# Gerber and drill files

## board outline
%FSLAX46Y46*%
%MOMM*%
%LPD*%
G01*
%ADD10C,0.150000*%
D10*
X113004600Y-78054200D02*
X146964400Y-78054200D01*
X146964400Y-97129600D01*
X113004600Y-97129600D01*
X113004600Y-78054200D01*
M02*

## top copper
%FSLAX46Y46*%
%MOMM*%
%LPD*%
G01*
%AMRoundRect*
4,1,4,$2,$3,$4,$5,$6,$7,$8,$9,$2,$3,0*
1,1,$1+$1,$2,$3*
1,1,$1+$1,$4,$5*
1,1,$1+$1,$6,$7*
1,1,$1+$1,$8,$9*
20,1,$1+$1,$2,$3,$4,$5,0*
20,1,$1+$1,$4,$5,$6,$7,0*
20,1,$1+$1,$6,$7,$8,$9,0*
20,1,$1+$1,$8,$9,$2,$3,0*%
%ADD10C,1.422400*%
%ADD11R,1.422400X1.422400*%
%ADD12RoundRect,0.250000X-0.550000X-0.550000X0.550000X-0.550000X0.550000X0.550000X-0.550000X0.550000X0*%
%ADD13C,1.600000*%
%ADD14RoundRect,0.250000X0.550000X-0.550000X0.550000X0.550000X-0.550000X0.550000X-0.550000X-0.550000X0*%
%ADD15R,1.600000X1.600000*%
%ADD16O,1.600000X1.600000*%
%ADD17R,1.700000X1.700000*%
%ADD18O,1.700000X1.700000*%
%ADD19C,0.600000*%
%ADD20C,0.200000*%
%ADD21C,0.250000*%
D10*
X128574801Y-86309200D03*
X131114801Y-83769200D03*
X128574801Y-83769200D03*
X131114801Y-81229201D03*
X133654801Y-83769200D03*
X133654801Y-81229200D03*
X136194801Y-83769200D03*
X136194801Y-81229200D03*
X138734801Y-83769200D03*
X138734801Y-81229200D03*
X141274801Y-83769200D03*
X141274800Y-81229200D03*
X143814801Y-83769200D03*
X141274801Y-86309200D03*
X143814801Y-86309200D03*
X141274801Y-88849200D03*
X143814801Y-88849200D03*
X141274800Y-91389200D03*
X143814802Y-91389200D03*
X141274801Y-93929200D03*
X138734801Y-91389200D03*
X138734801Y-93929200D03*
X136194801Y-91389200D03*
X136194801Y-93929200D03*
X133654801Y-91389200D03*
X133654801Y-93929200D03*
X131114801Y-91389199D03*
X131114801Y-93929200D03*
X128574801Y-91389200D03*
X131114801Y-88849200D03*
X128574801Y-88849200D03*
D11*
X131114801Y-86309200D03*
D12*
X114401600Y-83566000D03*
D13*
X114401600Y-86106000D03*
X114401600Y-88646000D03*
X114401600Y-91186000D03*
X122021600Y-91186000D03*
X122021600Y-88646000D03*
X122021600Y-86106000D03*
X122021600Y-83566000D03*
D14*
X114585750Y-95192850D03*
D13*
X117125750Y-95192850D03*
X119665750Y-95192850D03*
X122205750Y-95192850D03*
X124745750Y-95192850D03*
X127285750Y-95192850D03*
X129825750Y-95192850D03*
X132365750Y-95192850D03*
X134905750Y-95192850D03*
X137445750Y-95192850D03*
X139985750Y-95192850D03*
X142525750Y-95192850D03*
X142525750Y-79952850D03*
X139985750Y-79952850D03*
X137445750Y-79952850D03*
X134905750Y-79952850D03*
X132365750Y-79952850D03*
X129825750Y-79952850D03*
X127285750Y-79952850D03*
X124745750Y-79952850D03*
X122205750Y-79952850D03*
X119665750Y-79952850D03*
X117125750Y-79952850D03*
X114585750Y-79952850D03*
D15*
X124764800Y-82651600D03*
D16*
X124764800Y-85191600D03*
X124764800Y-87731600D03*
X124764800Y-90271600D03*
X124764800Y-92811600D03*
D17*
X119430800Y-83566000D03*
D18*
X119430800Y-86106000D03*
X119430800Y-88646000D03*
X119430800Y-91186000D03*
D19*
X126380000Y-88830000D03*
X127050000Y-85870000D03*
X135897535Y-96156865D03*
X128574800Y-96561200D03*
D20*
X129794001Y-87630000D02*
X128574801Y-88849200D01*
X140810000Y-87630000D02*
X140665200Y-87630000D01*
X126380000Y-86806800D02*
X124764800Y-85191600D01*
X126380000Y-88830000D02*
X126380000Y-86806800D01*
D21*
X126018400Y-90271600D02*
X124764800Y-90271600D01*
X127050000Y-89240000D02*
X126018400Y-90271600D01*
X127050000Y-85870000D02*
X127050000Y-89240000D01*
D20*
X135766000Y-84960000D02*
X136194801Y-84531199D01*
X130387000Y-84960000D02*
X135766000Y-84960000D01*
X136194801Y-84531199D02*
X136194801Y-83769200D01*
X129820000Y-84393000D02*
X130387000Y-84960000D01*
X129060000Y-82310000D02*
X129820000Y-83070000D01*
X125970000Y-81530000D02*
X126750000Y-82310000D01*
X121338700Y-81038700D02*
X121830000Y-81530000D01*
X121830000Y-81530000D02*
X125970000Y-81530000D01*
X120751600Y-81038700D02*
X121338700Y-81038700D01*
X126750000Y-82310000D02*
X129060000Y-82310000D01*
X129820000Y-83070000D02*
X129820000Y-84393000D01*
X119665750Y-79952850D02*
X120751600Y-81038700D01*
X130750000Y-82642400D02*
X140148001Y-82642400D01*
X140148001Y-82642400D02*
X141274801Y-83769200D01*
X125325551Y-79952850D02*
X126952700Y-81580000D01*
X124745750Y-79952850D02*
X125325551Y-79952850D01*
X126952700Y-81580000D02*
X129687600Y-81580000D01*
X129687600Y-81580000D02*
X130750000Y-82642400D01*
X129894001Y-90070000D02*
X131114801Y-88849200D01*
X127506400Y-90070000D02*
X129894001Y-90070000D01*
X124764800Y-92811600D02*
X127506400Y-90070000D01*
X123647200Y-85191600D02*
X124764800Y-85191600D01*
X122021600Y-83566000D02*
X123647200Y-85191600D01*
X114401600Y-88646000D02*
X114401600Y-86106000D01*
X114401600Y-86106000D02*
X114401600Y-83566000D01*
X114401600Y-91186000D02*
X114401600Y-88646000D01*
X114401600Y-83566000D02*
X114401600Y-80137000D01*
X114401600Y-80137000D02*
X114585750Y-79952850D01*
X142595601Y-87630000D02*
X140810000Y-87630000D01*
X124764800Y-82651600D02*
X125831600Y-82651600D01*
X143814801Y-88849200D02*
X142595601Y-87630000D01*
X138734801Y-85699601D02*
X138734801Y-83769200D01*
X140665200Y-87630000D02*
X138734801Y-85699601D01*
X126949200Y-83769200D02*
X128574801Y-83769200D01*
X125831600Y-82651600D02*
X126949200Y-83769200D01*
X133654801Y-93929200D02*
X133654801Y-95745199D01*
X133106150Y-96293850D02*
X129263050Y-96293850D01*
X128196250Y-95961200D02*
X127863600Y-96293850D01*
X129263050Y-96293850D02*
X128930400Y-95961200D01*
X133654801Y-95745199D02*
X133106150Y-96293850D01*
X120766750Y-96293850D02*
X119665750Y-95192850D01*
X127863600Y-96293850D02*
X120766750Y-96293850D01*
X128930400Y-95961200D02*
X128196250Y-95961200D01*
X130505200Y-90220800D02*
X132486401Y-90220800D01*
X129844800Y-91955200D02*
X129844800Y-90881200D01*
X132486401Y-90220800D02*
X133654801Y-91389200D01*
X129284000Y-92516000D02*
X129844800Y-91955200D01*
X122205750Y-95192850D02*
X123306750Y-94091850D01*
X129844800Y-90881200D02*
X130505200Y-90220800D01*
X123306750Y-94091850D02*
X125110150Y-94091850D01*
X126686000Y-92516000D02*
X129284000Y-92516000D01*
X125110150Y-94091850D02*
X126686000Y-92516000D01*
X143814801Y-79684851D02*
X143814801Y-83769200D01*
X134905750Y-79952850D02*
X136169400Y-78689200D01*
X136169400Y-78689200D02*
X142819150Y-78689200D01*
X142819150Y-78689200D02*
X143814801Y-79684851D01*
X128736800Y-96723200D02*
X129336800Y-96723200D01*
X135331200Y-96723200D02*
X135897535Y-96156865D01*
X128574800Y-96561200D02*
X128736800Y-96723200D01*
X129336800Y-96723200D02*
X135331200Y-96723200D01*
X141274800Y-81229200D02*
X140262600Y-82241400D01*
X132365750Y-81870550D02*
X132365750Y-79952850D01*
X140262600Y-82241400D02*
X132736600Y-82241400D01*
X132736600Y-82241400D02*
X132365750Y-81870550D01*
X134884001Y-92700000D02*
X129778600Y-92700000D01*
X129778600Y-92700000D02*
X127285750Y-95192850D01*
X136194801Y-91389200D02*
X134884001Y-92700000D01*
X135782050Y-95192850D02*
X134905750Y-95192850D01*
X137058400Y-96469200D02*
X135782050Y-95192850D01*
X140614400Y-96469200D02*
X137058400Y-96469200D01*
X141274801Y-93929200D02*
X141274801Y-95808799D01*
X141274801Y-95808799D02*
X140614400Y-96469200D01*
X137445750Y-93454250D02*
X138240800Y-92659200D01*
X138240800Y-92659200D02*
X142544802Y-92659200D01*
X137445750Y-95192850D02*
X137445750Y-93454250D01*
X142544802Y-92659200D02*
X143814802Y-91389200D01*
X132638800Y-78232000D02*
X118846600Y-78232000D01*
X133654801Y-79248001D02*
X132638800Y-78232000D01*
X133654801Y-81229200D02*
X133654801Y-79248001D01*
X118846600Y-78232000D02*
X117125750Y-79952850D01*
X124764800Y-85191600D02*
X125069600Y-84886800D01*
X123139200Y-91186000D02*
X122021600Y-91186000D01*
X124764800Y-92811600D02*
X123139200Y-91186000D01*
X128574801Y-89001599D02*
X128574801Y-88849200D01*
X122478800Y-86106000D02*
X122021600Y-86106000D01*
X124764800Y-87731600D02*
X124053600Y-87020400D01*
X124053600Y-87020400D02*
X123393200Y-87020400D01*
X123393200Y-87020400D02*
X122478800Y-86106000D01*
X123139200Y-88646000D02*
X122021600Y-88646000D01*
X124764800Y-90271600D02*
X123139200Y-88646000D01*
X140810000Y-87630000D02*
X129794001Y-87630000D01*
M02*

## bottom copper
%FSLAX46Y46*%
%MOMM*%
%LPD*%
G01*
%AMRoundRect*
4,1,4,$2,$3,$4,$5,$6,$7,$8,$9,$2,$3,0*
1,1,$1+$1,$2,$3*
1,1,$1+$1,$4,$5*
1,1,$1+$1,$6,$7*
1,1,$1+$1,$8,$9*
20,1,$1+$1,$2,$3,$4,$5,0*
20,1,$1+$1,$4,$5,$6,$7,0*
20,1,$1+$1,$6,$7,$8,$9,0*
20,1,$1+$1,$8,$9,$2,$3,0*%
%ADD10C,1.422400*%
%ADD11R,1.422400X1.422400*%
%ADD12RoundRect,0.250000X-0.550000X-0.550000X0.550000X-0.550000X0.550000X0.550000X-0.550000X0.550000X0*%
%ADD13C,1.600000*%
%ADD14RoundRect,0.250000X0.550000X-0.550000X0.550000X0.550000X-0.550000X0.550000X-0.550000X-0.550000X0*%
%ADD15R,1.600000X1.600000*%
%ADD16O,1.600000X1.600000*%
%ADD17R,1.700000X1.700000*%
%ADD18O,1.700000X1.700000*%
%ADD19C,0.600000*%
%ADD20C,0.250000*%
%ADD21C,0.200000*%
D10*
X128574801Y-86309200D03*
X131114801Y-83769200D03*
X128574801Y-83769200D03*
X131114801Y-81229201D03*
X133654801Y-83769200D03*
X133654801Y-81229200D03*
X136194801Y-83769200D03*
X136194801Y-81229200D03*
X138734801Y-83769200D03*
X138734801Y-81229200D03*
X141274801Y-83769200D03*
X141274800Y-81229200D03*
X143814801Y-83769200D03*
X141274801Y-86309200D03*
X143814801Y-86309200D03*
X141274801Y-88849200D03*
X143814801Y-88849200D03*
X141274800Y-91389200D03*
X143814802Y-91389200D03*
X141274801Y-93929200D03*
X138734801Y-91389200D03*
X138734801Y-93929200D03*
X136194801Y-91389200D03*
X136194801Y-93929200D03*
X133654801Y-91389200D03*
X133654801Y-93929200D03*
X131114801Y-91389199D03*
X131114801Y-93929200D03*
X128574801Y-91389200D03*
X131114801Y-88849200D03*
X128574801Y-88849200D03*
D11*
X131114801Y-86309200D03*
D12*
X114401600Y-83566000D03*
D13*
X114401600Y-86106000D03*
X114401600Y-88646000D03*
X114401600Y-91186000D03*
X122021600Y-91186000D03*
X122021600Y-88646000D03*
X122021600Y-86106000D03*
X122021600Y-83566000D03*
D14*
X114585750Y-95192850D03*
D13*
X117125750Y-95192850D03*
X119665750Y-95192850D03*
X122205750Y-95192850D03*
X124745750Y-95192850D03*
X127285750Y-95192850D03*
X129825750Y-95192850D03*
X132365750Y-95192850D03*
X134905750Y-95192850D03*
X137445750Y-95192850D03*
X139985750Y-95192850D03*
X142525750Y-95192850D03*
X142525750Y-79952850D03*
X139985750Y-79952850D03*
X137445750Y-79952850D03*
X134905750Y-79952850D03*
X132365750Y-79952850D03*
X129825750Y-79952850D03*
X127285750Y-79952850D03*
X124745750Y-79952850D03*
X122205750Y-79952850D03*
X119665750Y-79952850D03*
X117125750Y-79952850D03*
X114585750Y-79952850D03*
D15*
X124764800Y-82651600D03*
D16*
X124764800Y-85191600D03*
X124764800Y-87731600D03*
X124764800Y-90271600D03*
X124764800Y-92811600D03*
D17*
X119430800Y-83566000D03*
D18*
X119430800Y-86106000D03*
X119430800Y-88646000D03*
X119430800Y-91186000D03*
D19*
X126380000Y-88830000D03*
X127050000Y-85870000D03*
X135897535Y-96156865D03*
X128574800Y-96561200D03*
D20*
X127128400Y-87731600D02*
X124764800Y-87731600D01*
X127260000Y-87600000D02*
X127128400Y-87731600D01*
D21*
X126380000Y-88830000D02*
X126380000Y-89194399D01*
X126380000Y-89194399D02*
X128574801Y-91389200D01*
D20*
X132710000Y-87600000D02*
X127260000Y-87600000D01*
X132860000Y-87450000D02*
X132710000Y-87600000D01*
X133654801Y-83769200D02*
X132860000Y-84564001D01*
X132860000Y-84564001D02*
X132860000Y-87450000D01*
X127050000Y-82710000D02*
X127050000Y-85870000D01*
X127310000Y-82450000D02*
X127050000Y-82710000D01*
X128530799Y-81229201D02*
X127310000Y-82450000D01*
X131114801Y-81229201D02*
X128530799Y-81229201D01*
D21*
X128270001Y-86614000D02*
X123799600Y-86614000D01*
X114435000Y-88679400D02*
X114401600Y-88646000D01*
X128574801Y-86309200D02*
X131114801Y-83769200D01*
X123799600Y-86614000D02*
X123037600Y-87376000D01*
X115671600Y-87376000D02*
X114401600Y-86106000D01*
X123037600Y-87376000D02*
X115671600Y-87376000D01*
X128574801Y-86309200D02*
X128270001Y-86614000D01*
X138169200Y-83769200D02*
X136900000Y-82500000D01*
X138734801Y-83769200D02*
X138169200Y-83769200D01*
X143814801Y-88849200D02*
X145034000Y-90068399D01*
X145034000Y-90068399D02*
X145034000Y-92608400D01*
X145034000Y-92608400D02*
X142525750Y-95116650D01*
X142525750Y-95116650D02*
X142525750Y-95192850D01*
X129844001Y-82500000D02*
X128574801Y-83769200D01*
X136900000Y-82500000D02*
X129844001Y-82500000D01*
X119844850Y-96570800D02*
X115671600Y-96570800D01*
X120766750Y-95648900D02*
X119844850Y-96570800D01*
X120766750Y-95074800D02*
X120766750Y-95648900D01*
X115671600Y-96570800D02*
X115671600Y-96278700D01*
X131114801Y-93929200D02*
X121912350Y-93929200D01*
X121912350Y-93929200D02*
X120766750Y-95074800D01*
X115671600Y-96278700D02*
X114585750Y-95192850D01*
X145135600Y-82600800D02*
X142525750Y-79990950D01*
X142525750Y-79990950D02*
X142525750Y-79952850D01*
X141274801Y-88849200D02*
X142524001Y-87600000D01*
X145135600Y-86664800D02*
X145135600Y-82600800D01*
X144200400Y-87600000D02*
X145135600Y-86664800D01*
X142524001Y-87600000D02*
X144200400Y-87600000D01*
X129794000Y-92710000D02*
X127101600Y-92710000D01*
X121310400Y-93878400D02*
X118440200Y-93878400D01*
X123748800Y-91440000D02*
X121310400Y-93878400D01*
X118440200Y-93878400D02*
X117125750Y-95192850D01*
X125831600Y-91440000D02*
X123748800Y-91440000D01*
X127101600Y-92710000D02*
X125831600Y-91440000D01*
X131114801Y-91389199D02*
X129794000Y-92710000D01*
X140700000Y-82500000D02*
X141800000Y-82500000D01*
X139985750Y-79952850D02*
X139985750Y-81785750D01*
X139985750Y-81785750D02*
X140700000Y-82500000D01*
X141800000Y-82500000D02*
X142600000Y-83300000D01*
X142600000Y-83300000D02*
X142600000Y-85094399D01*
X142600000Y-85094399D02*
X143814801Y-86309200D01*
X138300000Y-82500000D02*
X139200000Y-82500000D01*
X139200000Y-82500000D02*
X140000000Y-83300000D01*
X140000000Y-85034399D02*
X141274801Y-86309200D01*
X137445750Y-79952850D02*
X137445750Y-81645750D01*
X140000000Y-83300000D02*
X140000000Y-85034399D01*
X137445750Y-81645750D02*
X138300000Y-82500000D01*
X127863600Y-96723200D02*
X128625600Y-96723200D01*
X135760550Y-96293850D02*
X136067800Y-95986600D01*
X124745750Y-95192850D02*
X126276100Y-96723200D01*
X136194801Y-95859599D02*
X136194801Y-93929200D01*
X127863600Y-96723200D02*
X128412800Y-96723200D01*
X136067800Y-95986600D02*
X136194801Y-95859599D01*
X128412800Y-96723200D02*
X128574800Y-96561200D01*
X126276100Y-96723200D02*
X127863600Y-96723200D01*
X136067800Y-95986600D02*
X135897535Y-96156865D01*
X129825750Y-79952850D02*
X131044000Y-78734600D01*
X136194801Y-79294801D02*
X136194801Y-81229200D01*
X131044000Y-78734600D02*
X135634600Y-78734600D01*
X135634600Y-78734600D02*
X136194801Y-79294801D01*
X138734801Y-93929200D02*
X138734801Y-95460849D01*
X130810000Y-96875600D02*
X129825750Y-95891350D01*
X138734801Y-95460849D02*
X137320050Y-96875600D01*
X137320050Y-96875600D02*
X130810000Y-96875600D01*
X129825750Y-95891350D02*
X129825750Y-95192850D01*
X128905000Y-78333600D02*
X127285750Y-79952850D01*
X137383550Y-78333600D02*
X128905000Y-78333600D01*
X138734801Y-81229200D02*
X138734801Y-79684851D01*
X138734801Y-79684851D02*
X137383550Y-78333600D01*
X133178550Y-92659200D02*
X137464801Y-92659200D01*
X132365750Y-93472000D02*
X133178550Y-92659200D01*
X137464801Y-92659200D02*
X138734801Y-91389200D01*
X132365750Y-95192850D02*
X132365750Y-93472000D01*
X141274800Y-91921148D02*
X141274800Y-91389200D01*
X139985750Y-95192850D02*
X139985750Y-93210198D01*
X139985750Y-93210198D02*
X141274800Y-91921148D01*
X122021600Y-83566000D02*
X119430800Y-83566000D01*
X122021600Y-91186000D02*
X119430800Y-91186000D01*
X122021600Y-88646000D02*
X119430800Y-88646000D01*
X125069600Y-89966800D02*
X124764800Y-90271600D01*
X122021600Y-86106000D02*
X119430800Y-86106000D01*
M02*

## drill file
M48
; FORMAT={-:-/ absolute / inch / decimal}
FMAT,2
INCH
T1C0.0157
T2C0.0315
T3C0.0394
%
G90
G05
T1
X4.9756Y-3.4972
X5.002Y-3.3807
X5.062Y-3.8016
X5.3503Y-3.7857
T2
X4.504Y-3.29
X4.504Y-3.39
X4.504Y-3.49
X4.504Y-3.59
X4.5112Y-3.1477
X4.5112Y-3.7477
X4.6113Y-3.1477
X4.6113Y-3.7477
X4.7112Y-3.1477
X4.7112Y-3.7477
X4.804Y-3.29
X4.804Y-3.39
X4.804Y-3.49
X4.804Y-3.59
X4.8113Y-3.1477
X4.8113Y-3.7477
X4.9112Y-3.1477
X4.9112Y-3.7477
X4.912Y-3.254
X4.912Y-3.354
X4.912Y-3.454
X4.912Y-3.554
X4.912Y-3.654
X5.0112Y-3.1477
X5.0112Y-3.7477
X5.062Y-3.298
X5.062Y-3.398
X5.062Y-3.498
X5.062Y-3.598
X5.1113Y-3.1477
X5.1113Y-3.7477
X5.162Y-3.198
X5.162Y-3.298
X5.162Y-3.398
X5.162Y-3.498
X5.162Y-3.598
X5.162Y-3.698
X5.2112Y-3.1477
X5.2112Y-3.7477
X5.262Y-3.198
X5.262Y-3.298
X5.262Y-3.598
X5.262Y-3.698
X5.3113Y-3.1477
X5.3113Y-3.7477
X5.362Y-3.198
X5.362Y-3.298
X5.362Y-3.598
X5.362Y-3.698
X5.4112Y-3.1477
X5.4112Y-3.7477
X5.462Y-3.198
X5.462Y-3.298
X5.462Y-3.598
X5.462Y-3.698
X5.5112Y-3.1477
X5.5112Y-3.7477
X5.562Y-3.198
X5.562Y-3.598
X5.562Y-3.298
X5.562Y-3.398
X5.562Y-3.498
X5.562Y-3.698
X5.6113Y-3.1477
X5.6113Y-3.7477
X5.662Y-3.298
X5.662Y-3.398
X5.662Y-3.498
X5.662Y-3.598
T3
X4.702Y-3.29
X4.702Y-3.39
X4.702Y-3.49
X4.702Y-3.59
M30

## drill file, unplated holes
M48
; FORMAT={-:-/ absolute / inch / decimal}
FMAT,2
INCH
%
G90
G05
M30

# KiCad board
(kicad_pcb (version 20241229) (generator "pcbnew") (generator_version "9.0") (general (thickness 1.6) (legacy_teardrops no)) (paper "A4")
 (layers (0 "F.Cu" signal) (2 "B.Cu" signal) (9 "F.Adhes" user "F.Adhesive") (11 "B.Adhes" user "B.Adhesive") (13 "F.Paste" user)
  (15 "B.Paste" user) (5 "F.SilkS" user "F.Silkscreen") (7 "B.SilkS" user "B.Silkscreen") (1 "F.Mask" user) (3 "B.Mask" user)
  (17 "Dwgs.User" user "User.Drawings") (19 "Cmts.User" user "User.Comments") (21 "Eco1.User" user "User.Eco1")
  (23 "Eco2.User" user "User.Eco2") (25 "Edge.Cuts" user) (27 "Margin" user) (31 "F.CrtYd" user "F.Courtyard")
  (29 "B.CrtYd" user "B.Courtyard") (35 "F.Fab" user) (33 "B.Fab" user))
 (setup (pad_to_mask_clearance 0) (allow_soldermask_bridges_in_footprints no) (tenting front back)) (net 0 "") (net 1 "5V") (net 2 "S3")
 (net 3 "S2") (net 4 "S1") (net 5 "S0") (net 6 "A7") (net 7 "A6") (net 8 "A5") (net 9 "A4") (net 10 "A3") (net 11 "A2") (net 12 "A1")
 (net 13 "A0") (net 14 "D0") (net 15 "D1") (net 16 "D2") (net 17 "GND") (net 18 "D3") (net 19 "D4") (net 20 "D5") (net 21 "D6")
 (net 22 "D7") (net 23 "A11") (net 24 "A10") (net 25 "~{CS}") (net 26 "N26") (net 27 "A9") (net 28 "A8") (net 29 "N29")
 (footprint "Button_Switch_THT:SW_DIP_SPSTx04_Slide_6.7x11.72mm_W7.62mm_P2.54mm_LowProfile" (layer "F.Cu") (at 114.4016 83.566)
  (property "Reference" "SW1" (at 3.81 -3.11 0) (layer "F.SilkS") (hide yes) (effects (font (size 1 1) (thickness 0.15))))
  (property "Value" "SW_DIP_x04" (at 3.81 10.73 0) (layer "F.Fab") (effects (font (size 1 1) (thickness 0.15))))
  (pad "1" thru_hole roundrect (at 0 0) (size 1.6 1.6) (drill 0.8) (layers "*.Cu" "*.Mask") (remove_unused_layers no)
   (roundrect_rratio 0.15625) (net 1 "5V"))
  (pad "2" thru_hole circle (at 0 2.54) (size 1.6 1.6) (drill 0.8) (layers "*.Cu" "*.Mask") (remove_unused_layers no) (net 1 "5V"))
  (pad "3" thru_hole circle (at 0 5.08) (size 1.6 1.6) (drill 0.8) (layers "*.Cu" "*.Mask") (remove_unused_layers no) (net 1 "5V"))
  (pad "4" thru_hole circle (at 0 7.62) (size 1.6 1.6) (drill 0.8) (layers "*.Cu" "*.Mask") (remove_unused_layers no) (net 1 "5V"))
  (pad "5" thru_hole circle (at 7.62 7.62) (size 1.6 1.6) (drill 0.8) (layers "*.Cu" "*.Mask") (remove_unused_layers no) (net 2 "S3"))
  (pad "6" thru_hole circle (at 7.62 5.08) (size 1.6 1.6) (drill 0.8) (layers "*.Cu" "*.Mask") (remove_unused_layers no) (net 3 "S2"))
  (pad "7" thru_hole circle (at 7.62 2.54) (size 1.6 1.6) (drill 0.8) (layers "*.Cu" "*.Mask") (remove_unused_layers no) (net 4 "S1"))
  (pad "8" thru_hole circle (at 7.62 0) (size 1.6 1.6) (drill 0.8) (layers "*.Cu" "*.Mask") (remove_unused_layers no) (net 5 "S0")))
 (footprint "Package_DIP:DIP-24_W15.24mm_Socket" (layer "F.Cu") (at 114.58575 95.19285 90)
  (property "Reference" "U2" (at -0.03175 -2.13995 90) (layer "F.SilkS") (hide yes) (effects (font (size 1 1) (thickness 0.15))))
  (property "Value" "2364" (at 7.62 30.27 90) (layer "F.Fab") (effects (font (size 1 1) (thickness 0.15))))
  (pad "1" thru_hole roundrect (at 0 0 90) (size 1.6 1.6) (drill 0.8) (layers "*.Cu" "*.Mask") (remove_unused_layers no)
   (roundrect_rratio 0.15625) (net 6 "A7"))
  (pad "2" thru_hole circle (at 0 2.54 90) (size 1.6 1.6) (drill 0.8) (layers "*.Cu" "*.Mask") (remove_unused_layers no) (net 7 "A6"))
  (pad "3" thru_hole circle (at 0 5.08 90) (size 1.6 1.6) (drill 0.8) (layers "*.Cu" "*.Mask") (remove_unused_layers no) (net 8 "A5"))
  (pad "4" thru_hole circle (at 0 7.62 90) (size 1.6 1.6) (drill 0.8) (layers "*.Cu" "*.Mask") (remove_unused_layers no) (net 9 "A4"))
  (pad "5" thru_hole circle (at 0 10.16 90) (size 1.6 1.6) (drill 0.8) (layers "*.Cu" "*.Mask") (remove_unused_layers no) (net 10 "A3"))
  (pad "6" thru_hole circle (at 0 12.7 90) (size 1.6 1.6) (drill 0.8) (layers "*.Cu" "*.Mask") (remove_unused_layers no) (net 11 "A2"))
  (pad "7" thru_hole circle (at 0 15.24 90) (size 1.6 1.6) (drill 0.8) (layers "*.Cu" "*.Mask") (remove_unused_layers no) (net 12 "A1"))
  (pad "8" thru_hole circle (at 0 17.78 90) (size 1.6 1.6) (drill 0.8) (layers "*.Cu" "*.Mask") (remove_unused_layers no) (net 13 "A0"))
  (pad "9" thru_hole circle (at 0 20.32 90) (size 1.6 1.6) (drill 0.8) (layers "*.Cu" "*.Mask") (remove_unused_layers no) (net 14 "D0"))
  (pad "10" thru_hole circle (at 0 22.86 90) (size 1.6 1.6) (drill 0.8) (layers "*.Cu" "*.Mask") (remove_unused_layers no) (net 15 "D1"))
  (pad "11" thru_hole circle (at 0 25.4 90) (size 1.6 1.6) (drill 0.8) (layers "*.Cu" "*.Mask") (remove_unused_layers no) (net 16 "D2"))
  (pad "12" thru_hole circle (at 0 27.94 90) (size 1.6 1.6) (drill 0.8) (layers "*.Cu" "*.Mask") (remove_unused_layers no) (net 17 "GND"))
  (pad "13" thru_hole circle (at 15.24 27.94 90) (size 1.6 1.6) (drill 0.8) (layers "*.Cu" "*.Mask") (remove_unused_layers no) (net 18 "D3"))
  (pad "14" thru_hole circle (at 15.24 25.4 90) (size 1.6 1.6) (drill 0.8) (layers "*.Cu" "*.Mask") (remove_unused_layers no) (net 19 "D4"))
  (pad "15" thru_hole circle (at 15.24 22.86 90) (size 1.6 1.6) (drill 0.8) (layers "*.Cu" "*.Mask") (remove_unused_layers no) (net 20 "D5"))
  (pad "16" thru_hole circle (at 15.24 20.32 90) (size 1.6 1.6) (drill 0.8) (layers "*.Cu" "*.Mask") (remove_unused_layers no) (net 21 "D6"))
  (pad "17" thru_hole circle (at 15.24 17.78 90) (size 1.6 1.6) (drill 0.8) (layers "*.Cu" "*.Mask") (remove_unused_layers no) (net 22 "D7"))
  (pad "18" thru_hole circle (at 15.24 15.24 90) (size 1.6 1.6) (drill 0.8) (layers "*.Cu" "*.Mask") (remove_unused_layers no)
   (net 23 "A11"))
  (pad "19" thru_hole circle (at 15.24 12.7 90) (size 1.6 1.6) (drill 0.8) (layers "*.Cu" "*.Mask") (remove_unused_layers no) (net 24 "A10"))
  (pad "20" thru_hole circle (at 15.24 10.16 90) (size 1.6 1.6) (drill 0.8) (layers "*.Cu" "*.Mask") (remove_unused_layers no)
   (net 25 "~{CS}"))
  (pad "21" thru_hole circle (at 15.24 7.62 90) (size 1.6 1.6) (drill 0.8) (layers "*.Cu" "*.Mask") (remove_unused_layers no) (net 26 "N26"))
  (pad "22" thru_hole circle (at 15.24 5.08 90) (size 1.6 1.6) (drill 0.8) (layers "*.Cu" "*.Mask") (remove_unused_layers no) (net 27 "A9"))
  (pad "23" thru_hole circle (at 15.24 2.54 90) (size 1.6 1.6) (drill 0.8) (layers "*.Cu" "*.Mask") (remove_unused_layers no) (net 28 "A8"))
  (pad "24" thru_hole circle (at 15.24 0 90) (size 1.6 1.6) (drill 0.8) (layers "*.Cu" "*.Mask") (remove_unused_layers no) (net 1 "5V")))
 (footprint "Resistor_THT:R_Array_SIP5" (layer "F.Cu") (at 124.7648 82.6516 -90)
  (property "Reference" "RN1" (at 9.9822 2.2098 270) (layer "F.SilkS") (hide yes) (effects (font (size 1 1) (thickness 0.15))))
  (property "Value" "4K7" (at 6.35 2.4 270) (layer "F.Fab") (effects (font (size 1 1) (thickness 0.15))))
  (pad "1" thru_hole rect (at 0 0 270) (size 1.6 1.6) (drill 0.8) (layers "*.Cu" "*.Mask") (remove_unused_layers no) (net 17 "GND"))
  (pad "2" thru_hole oval (at 2.54 0 270) (size 1.6 1.6) (drill 0.8) (layers "*.Cu" "*.Mask") (remove_unused_layers no) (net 5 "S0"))
  (pad "3" thru_hole oval (at 5.08 0 270) (size 1.6 1.6) (drill 0.8) (layers "*.Cu" "*.Mask") (remove_unused_layers no) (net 4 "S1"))
  (pad "4" thru_hole oval (at 7.62 0 270) (size 1.6 1.6) (drill 0.8) (layers "*.Cu" "*.Mask") (remove_unused_layers no) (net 3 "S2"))
  (pad "5" thru_hole oval (at 10.16 0 270) (size 1.6 1.6) (drill 0.8) (layers "*.Cu" "*.Mask") (remove_unused_layers no) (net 2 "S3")))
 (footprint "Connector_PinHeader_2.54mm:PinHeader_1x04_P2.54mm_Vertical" (layer "F.Cu") (at 119.4308 83.566)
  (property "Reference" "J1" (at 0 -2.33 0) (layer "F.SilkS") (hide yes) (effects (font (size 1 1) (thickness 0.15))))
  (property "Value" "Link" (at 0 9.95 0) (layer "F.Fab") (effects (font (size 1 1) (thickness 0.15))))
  (pad "1" thru_hole rect (at 0 0) (size 1.7 1.7) (drill 1) (layers "*.Cu" "*.Mask") (remove_unused_layers no) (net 5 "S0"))
  (pad "2" thru_hole oval (at 0 2.54) (size 1.7 1.7) (drill 1) (layers "*.Cu" "*.Mask") (remove_unused_layers no) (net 4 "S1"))
  (pad "3" thru_hole oval (at 0 5.08) (size 1.7 1.7) (drill 1) (layers "*.Cu" "*.Mask") (remove_unused_layers no) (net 3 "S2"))
  (pad "4" thru_hole oval (at 0 7.62) (size 1.7 1.7) (drill 1) (layers "*.Cu" "*.Mask") (remove_unused_layers no) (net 2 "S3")))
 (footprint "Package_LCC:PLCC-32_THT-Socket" (layer "F.Cu") (at 131.114801 86.3092 90)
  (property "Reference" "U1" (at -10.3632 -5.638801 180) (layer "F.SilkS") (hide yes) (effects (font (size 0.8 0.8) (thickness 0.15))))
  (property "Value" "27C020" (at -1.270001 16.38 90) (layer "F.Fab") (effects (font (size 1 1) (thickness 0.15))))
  (pad "1" thru_hole rect (at 0 0 90) (size 1.4224 1.4224) (drill 0.8) (layers "*.Cu" "*.Mask") (remove_unused_layers no) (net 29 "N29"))
  (pad "2" thru_hole circle (at -2.54 -2.54 90) (size 1.4224 1.4224) (drill 0.8) (layers "*.Cu" "*.Mask") (remove_unused_layers no)
   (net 17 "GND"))
  (pad "3" thru_hole circle (at -2.54 0 90) (size 1.4224 1.4224) (drill 0.8) (layers "*.Cu" "*.Mask") (remove_unused_layers no) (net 2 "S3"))
  (pad "4" thru_hole circle (at -5.08 -2.54 90) (size 1.4224 1.4224) (drill 0.8) (layers "*.Cu" "*.Mask") (remove_unused_layers no)
   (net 5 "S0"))
  (pad "5" thru_hole circle (at -7.62 0 90) (size 1.4224 1.4224) (drill 0.8) (layers "*.Cu" "*.Mask") (remove_unused_layers no) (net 6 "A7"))
  (pad "6" thru_hole circle (at -5.079999 0 90) (size 1.4224 1.4224) (drill 0.8) (layers "*.Cu" "*.Mask") (remove_unused_layers no)
   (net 7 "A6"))
  (pad "7" thru_hole circle (at -7.62 2.54 90) (size 1.4224 1.4224) (drill 0.8) (layers "*.Cu" "*.Mask") (remove_unused_layers no)
   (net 8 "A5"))
  (pad "8" thru_hole circle (at -5.08 2.54 90) (size 1.4224 1.4224) (drill 0.8) (layers "*.Cu" "*.Mask") (remove_unused_layers no)
   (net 9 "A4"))
  (pad "9" thru_hole circle (at -7.62 5.08 90) (size 1.4224 1.4224) (drill 0.8) (layers "*.Cu" "*.Mask") (remove_unused_layers no)
   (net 10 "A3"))
  (pad "10" thru_hole circle (at -5.08 5.08 90) (size 1.4224 1.4224) (drill 0.8) (layers "*.Cu" "*.Mask") (remove_unused_layers no)
   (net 11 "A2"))
  (pad "11" thru_hole circle (at -7.62 7.62 90) (size 1.4224 1.4224) (drill 0.8) (layers "*.Cu" "*.Mask") (remove_unused_layers no)
   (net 12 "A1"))
  (pad "12" thru_hole circle (at -5.08 7.62 90) (size 1.4224 1.4224) (drill 0.8) (layers "*.Cu" "*.Mask") (remove_unused_layers no)
   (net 13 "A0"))
  (pad "13" thru_hole circle (at -7.62 10.16 90) (size 1.4224 1.4224) (drill 0.8) (layers "*.Cu" "*.Mask") (remove_unused_layers no)
   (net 14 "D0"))
  (pad "14" thru_hole circle (at -5.08 12.700001 90) (size 1.4224 1.4224) (drill 0.8) (layers "*.Cu" "*.Mask") (remove_unused_layers no)
   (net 15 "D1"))
  (pad "15" thru_hole circle (at -5.08 10.159999 90) (size 1.4224 1.4224) (drill 0.8) (layers "*.Cu" "*.Mask") (remove_unused_layers no)
   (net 16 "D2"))
  (pad "16" thru_hole circle (at -2.54 12.7 90) (size 1.4224 1.4224) (drill 0.8) (layers "*.Cu" "*.Mask") (remove_unused_layers no)
   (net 17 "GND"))
  (pad "17" thru_hole circle (at -2.54 10.16 90) (size 1.4224 1.4224) (drill 0.8) (layers "*.Cu" "*.Mask") (remove_unused_layers no)
   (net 18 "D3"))
  (pad "18" thru_hole circle (at 0 12.7 90) (size 1.4224 1.4224) (drill 0.8) (layers "*.Cu" "*.Mask") (remove_unused_layers no)
   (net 19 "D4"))
  (pad "19" thru_hole circle (at 0 10.16 90) (size 1.4224 1.4224) (drill 0.8) (layers "*.Cu" "*.Mask") (remove_unused_layers no)
   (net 20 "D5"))
  (pad "20" thru_hole circle (at 2.54 12.7 90) (size 1.4224 1.4224) (drill 0.8) (layers "*.Cu" "*.Mask") (remove_unused_layers no)
   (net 21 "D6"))
  (pad "21" thru_hole circle (at 5.08 10.159999 90) (size 1.4224 1.4224) (drill 0.8) (layers "*.Cu" "*.Mask") (remove_unused_layers no)
   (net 22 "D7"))
  (pad "22" thru_hole circle (at 2.54 10.16 90) (size 1.4224 1.4224) (drill 0.8) (layers "*.Cu" "*.Mask") (remove_unused_layers no)
   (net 25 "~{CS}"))
  (pad "23" thru_hole circle (at 5.08 7.62 90) (size 1.4224 1.4224) (drill 0.8) (layers "*.Cu" "*.Mask") (remove_unused_layers no)
   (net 24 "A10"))
  (pad "24" thru_hole circle (at 2.54 7.62 90) (size 1.4224 1.4224) (drill 0.8) (layers "*.Cu" "*.Mask") (remove_unused_layers no)
   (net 17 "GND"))
  (pad "25" thru_hole circle (at 5.08 5.08 90) (size 1.4224 1.4224) (drill 0.8) (layers "*.Cu" "*.Mask") (remove_unused_layers no)
   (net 23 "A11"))
  (pad "26" thru_hole circle (at 2.54 5.08 90) (size 1.4224 1.4224) (drill 0.8) (layers "*.Cu" "*.Mask") (remove_unused_layers no)
   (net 27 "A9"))
  (pad "27" thru_hole circle (at 5.08 2.54 90) (size 1.4224 1.4224) (drill 0.8) (layers "*.Cu" "*.Mask") (remove_unused_layers no)
   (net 28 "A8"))
  (pad "28" thru_hole circle (at 2.54 2.54 90) (size 1.4224 1.4224) (drill 0.8) (layers "*.Cu" "*.Mask") (remove_unused_layers no)
   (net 4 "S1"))
  (pad "29" thru_hole circle (at 5.079999 0 90) (size 1.4224 1.4224) (drill 0.8) (layers "*.Cu" "*.Mask") (remove_unused_layers no)
   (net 3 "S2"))
  (pad "30" thru_hole circle (at 2.54 -2.54 90) (size 1.4224 1.4224) (drill 0.8) (layers "*.Cu" "*.Mask") (remove_unused_layers no)
   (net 17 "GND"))
  (pad "31" thru_hole circle (at 2.54 0 90) (size 1.4224 1.4224) (drill 0.8) (layers "*.Cu" "*.Mask") (remove_unused_layers no) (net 1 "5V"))
  (pad "32" thru_hole circle (at 0 -2.54 90) (size 1.4224 1.4224) (drill 0.8) (layers "*.Cu" "*.Mask") (remove_unused_layers no)
   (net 1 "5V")))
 (gr_rect (start 113.0046 78.0542) (end 146.9644 97.1296) (stroke (width 0.15) (type default)) (fill no) (layer "Edge.Cuts"))
 (segment (start 124.74575 79.95285) (end 125.325551 79.95285) (width 0.2) (layer "F.Cu") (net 25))
 (segment (start 130.75 82.6424) (end 140.148001 82.6424) (width 0.2) (layer "F.Cu") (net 25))
 (segment (start 140.148001 82.6424) (end 141.274801 83.7692) (width 0.2) (layer "F.Cu") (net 25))
 (segment (start 125.325551 79.95285) (end 126.9527 81.58) (width 0.2) (layer "F.Cu") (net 25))
 (segment (start 126.9527 81.58) (end 129.6876 81.58) (width 0.2) (layer "F.Cu") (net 25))
 (segment (start 129.6876 81.58) (end 130.75 82.6424) (width 0.2) (layer "F.Cu") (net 25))
 (segment (start 114.4016 88.646) (end 114.4016 86.106) (width 0.2) (layer "F.Cu") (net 1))
 (segment (start 114.4016 86.106) (end 114.4016 83.566) (width 0.2) (layer "F.Cu") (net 1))
 (segment (start 114.4016 91.186) (end 114.4016 88.646) (width 0.2) (layer "F.Cu") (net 1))
 (segment (start 114.4016 83.566) (end 114.4016 80.137) (width 0.2) (layer "F.Cu") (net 1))
 (segment (start 114.4016 80.137) (end 114.58575 79.95285) (width 0.2) (layer "F.Cu") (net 1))
 (segment (start 128.270001 86.614) (end 123.7996 86.614) (width 0.2) (layer "B.Cu") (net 1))
 (segment (start 114.435 88.6794) (end 114.4016 88.646) (width 0.2) (layer "B.Cu") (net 1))
 (segment (start 128.574801 86.3092) (end 131.114801 83.7692) (width 0.2) (layer "B.Cu") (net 1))
 (segment (start 123.7996 86.614) (end 123.0376 87.376) (width 0.2) (layer "B.Cu") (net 1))
 (segment (start 115.6716 87.376) (end 114.4016 86.106) (width 0.2) (layer "B.Cu") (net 1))
 (segment (start 123.0376 87.376) (end 115.6716 87.376) (width 0.2) (layer "B.Cu") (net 1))
 (segment (start 128.574801 86.3092) (end 128.270001 86.614) (width 0.2) (layer "B.Cu") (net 1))
 (segment (start 142.595601 87.63) (end 140.81 87.63) (width 0.2) (layer "F.Cu") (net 17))
 (segment (start 124.7648 82.6516) (end 125.8316 82.6516) (width 0.2) (layer "F.Cu") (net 17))
 (segment (start 140.81 87.63) (end 140.6652 87.63) (width 0.2) (layer "F.Cu") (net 17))
 (segment (start 143.814801 88.8492) (end 142.595601 87.63) (width 0.2) (layer "F.Cu") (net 17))
 (segment (start 138.734801 85.699601) (end 138.734801 83.7692) (width 0.2) (layer "F.Cu") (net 17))
 (segment (start 140.6652 87.63) (end 138.734801 85.699601) (width 0.2) (layer "F.Cu") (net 17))
 (segment (start 126.9492 83.7692) (end 128.574801 83.7692) (width 0.2) (layer "F.Cu") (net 17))
 (segment (start 140.81 87.63) (end 129.794001 87.63) (width 0.2) (layer "F.Cu") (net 17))
 (segment (start 125.8316 82.6516) (end 126.9492 83.7692) (width 0.2) (layer "F.Cu") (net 17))
 (segment (start 129.794001 87.63) (end 128.574801 88.8492) (width 0.2) (layer "F.Cu") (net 17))
 (segment (start 128.574801 89.001599) (end 128.574801 88.8492) (width 0.2) (layer "F.Cu") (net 17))
 (segment (start 138.1692 83.7692) (end 136.9 82.5) (width 0.2) (layer "B.Cu") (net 17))
 (segment (start 138.734801 83.7692) (end 138.1692 83.7692) (width 0.2) (layer "B.Cu") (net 17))
 (segment (start 143.814801 88.8492) (end 145.034 90.068399) (width 0.2) (layer "B.Cu") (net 17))
 (segment (start 145.034 90.068399) (end 145.034 92.6084) (width 0.2) (layer "B.Cu") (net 17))
 (segment (start 145.034 92.6084) (end 142.52575 95.11665) (width 0.2) (layer "B.Cu") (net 17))
 (segment (start 142.52575 95.11665) (end 142.52575 95.19285) (width 0.2) (layer "B.Cu") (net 17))
 (segment (start 129.844001 82.5) (end 128.574801 83.7692) (width 0.2) (layer "B.Cu") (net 17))
 (segment (start 136.9 82.5) (end 129.844001 82.5) (width 0.2) (layer "B.Cu") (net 17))
 (segment (start 119.84485 96.5708) (end 115.6716 96.5708) (width 0.2) (layer "B.Cu") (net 6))
 (segment (start 120.76675 95.6489) (end 119.84485 96.5708) (width 0.2) (layer "B.Cu") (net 6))
 (segment (start 120.76675 95.0748) (end 120.76675 95.6489) (width 0.2) (layer "B.Cu") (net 6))
 (segment (start 115.6716 96.5708) (end 115.6716 96.2787) (width 0.2) (layer "B.Cu") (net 6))
 (segment (start 131.114801 93.9292) (end 121.91235 93.9292) (width 0.2) (layer "B.Cu") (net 6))
 (segment (start 121.91235 93.9292) (end 120.76675 95.0748) (width 0.2) (layer "B.Cu") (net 6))
 (segment (start 115.6716 96.2787) (end 114.58575 95.19285) (width 0.2) (layer "B.Cu") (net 6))
 (segment (start 145.1356 82.6008) (end 142.52575 79.99095) (width 0.2) (layer "B.Cu") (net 18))
 (segment (start 142.52575 79.99095) (end 142.52575 79.95285) (width 0.2) (layer "B.Cu") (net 18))
 (segment (start 141.274801 88.8492) (end 142.524001 87.6) (width 0.2) (layer "B.Cu") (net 18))
 (segment (start 145.1356 86.6648) (end 145.1356 82.6008) (width 0.2) (layer "B.Cu") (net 18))
 (segment (start 144.2004 87.6) (end 145.1356 86.6648) (width 0.2) (layer "B.Cu") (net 18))
 (segment (start 142.524001 87.6) (end 144.2004 87.6) (width 0.2) (layer "B.Cu") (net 18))
 (segment (start 129.794 92.71) (end 127.1016 92.71) (width 0.2) (layer "B.Cu") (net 7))
 (segment (start 121.3104 93.8784) (end 118.4402 93.8784) (width 0.2) (layer "B.Cu") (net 7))
 (segment (start 123.7488 91.44) (end 121.3104 93.8784) (width 0.2) (layer "B.Cu") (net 7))
 (segment (start 118.4402 93.8784) (end 117.12575 95.19285) (width 0.2) (layer "B.Cu") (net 7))
 (segment (start 125.8316 91.44) (end 123.7488 91.44) (width 0.2) (layer "B.Cu") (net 7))
 (segment (start 127.1016 92.71) (end 125.8316 91.44) (width 0.2) (layer "B.Cu") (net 7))
 (segment (start 131.114801 91.389199) (end 129.794 92.71) (width 0.2) (layer "B.Cu") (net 7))
 (segment (start 140.7 82.5) (end 141.8 82.5) (width 0.2) (layer "B.Cu") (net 19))
 (segment (start 139.98575 79.95285) (end 139.98575 81.78575) (width 0.2) (layer "B.Cu") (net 19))
 (segment (start 139.98575 81.78575) (end 140.7 82.5) (width 0.2) (layer "B.Cu") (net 19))
 (segment (start 141.8 82.5) (end 142.6 83.3) (width 0.2) (layer "B.Cu") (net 19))
 (segment (start 142.6 83.3) (end 142.6 85.094399) (width 0.2) (layer "B.Cu") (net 19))
 (segment (start 142.6 85.094399) (end 143.814801 86.3092) (width 0.2) (layer "B.Cu") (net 19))
 (segment (start 133.654801 93.9292) (end 133.654801 95.745199) (width 0.2) (layer "F.Cu") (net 8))
 (segment (start 133.10615 96.29385) (end 129.26305 96.29385) (width 0.2) (layer "F.Cu") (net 8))
 (segment (start 128.19625 95.9612) (end 127.8636 96.29385) (width 0.2) (layer "F.Cu") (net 8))
 (segment (start 129.26305 96.29385) (end 128.9304 95.9612) (width 0.2) (layer "F.Cu") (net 8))
 (segment (start 133.654801 95.745199) (end 133.10615 96.29385) (width 0.2) (layer "F.Cu") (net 8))
 (segment (start 120.76675 96.29385) (end 119.66575 95.19285) (width 0.2) (layer "F.Cu") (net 8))
 (segment (start 127.8636 96.29385) (end 120.76675 96.29385) (width 0.2) (layer "F.Cu") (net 8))
 (segment (start 128.9304 95.9612) (end 128.19625 95.9612) (width 0.2) (layer "F.Cu") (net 8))
 (segment (start 138.3 82.5) (end 139.2 82.5) (width 0.2) (layer "B.Cu") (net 20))
 (segment (start 139.2 82.5) (end 140 83.3) (width 0.2) (layer "B.Cu") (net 20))
 (segment (start 140 85.034399) (end 141.274801 86.3092) (width 0.2) (layer "B.Cu") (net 20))
 (segment (start 137.44575 79.95285) (end 137.44575 81.64575) (width 0.2) (layer "B.Cu") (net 20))
 (segment (start 140 83.3) (end 140 85.034399) (width 0.2) (layer "B.Cu") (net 20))
 (segment (start 137.44575 81.64575) (end 138.3 82.5) (width 0.2) (layer "B.Cu") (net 20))
 (segment (start 130.5052 90.2208) (end 132.486401 90.2208) (width 0.2) (layer "F.Cu") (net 9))
 (segment (start 129.8448 91.9552) (end 129.8448 90.8812) (width 0.2) (layer "F.Cu") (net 9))
 (segment (start 132.486401 90.2208) (end 133.654801 91.3892) (width 0.2) (layer "F.Cu") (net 9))
 (segment (start 129.284 92.516) (end 129.8448 91.9552) (width 0.2) (layer "F.Cu") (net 9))
 (segment (start 122.20575 95.19285) (end 123.30675 94.09185) (width 0.2) (layer "F.Cu") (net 9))
 (segment (start 129.8448 90.8812) (end 130.5052 90.2208) (width 0.2) (layer "F.Cu") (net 9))
 (segment (start 123.30675 94.09185) (end 125.11015 94.09185) (width 0.2) (layer "F.Cu") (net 9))
 (segment (start 126.686 92.516) (end 129.284 92.516) (width 0.2) (layer "F.Cu") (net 9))
 (segment (start 125.11015 94.09185) (end 126.686 92.516) (width 0.2) (layer "F.Cu") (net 9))
 (segment (start 143.814801 79.684851) (end 143.814801 83.7692) (width 0.2) (layer "F.Cu") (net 21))
 (segment (start 134.90575 79.95285) (end 136.1694 78.6892) (width 0.2) (layer "F.Cu") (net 21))
 (segment (start 136.1694 78.6892) (end 142.81915 78.6892) (width 0.2) (layer "F.Cu") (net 21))
 (segment (start 142.81915 78.6892) (end 143.814801 79.684851) (width 0.2) (layer "F.Cu") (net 21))
 (segment (start 128.7368 96.7232) (end 129.3368 96.7232) (width 0.2) (layer "F.Cu") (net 10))
 (segment (start 135.3312 96.7232) (end 135.897535 96.156865) (width 0.2) (layer "F.Cu") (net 10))
 (segment (start 128.5748 96.5612) (end 128.7368 96.7232) (width 0.2) (layer "F.Cu") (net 10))
 (segment (start 129.3368 96.7232) (end 135.3312 96.7232) (width 0.2) (layer "F.Cu") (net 10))
 (via (at 135.897535 96.156865) (size 0.6) (drill 0.4) (layers "F.Cu" "B.Cu") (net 10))
 (via (at 128.5748 96.5612) (size 0.6) (drill 0.4) (layers "F.Cu" "B.Cu") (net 10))
 (segment (start 127.8636 96.7232) (end 128.6256 96.7232) (width 0.2) (layer "B.Cu") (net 10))
 (segment (start 135.76055 96.29385) (end 136.0678 95.9866) (width 0.2) (layer "B.Cu") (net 10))
 (segment (start 124.74575 95.19285) (end 126.2761 96.7232) (width 0.2) (layer "B.Cu") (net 10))
 (segment (start 136.194801 95.859599) (end 136.194801 93.9292) (width 0.2) (layer "B.Cu") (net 10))
 (segment (start 127.8636 96.7232) (end 128.4128 96.7232) (width 0.2) (layer "B.Cu") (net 10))
 (segment (start 136.0678 95.9866) (end 136.194801 95.859599) (width 0.2) (layer "B.Cu") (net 10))
 (segment (start 128.4128 96.7232) (end 128.5748 96.5612) (width 0.2) (layer "B.Cu") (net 10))
 (segment (start 126.2761 96.7232) (end 127.8636 96.7232) (width 0.2) (layer "B.Cu") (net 10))
 (segment (start 136.0678 95.9866) (end 135.897535 96.156865) (width 0.2) (layer "B.Cu") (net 10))
 (segment (start 141.2748 81.2292) (end 140.2626 82.2414) (width 0.2) (layer "F.Cu") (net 22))
 (segment (start 132.36575 81.87055) (end 132.36575 79.95285) (width 0.2) (layer "F.Cu") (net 22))
 (segment (start 140.2626 82.2414) (end 132.7366 82.2414) (width 0.2) (layer "F.Cu") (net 22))
 (segment (start 132.7366 82.2414) (end 132.36575 81.87055) (width 0.2) (layer "F.Cu") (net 22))
 (segment (start 134.884001 92.7) (end 129.7786 92.7) (width 0.2) (layer "F.Cu") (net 11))
 (segment (start 129.7786 92.7) (end 127.28575 95.19285) (width 0.2) (layer "F.Cu") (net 11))
 (segment (start 136.194801 91.3892) (end 134.884001 92.7) (width 0.2) (layer "F.Cu") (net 11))
 (segment (start 129.82575 79.95285) (end 131.044 78.7346) (width 0.2) (layer "B.Cu") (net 23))
 (segment (start 136.194801 79.294801) (end 136.194801 81.2292) (width 0.2) (layer "B.Cu") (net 23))
 (segment (start 131.044 78.7346) (end 135.6346 78.7346) (width 0.2) (layer "B.Cu") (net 23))
 (segment (start 135.6346 78.7346) (end 136.194801 79.294801) (width 0.2) (layer "B.Cu") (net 23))
 (segment (start 138.734801 93.9292) (end 138.734801 95.460849) (width 0.2) (layer "B.Cu") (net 12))
 (segment (start 130.81 96.8756) (end 129.82575 95.89135) (width 0.2) (layer "B.Cu") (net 12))
 (segment (start 138.734801 95.460849) (end 137.32005 96.8756) (width 0.2) (layer "B.Cu") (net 12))
 (segment (start 137.32005 96.8756) (end 130.81 96.8756) (width 0.2) (layer "B.Cu") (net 12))
 (segment (start 129.82575 95.89135) (end 129.82575 95.19285) (width 0.2) (layer "B.Cu") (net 12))
 (segment (start 128.905 78.3336) (end 127.28575 79.95285) (width 0.2) (layer "B.Cu") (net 24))
 (segment (start 137.38355 78.3336) (end 128.905 78.3336) (width 0.2) (layer "B.Cu") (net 24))
 (segment (start 138.734801 81.2292) (end 138.734801 79.684851) (width 0.2) (layer "B.Cu") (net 24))
 (segment (start 138.734801 79.684851) (end 137.38355 78.3336) (width 0.2) (layer "B.Cu") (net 24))
 (segment (start 133.17855 92.6592) (end 137.464801 92.6592) (width 0.2) (layer "B.Cu") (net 13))
 (segment (start 132.36575 93.472) (end 133.17855 92.6592) (width 0.2) (layer "B.Cu") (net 13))
 (segment (start 137.464801 92.6592) (end 138.734801 91.3892) (width 0.2) (layer "B.Cu") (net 13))
 (segment (start 132.36575 95.19285) (end 132.36575 93.472) (width 0.2) (layer "B.Cu") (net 13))
 (segment (start 135.78205 95.19285) (end 134.90575 95.19285) (width 0.2) (layer "F.Cu") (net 14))
 (segment (start 137.0584 96.4692) (end 135.78205 95.19285) (width 0.2) (layer "F.Cu") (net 14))
 (segment (start 140.6144 96.4692) (end 137.0584 96.4692) (width 0.2) (layer "F.Cu") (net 14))
 (segment (start 141.274801 93.9292) (end 141.274801 95.808799) (width 0.2) (layer "F.Cu") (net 14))
 (segment (start 141.274801 95.808799) (end 140.6144 96.4692) (width 0.2) (layer "F.Cu") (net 14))
 (segment (start 137.44575 93.45425) (end 138.2408 92.6592) (width 0.2) (layer "F.Cu") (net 15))
 (segment (start 138.2408 92.6592) (end 142.544802 92.6592) (width 0.2) (layer "F.Cu") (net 15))
 (segment (start 137.44575 95.19285) (end 137.44575 93.45425) (width 0.2) (layer "F.Cu") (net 15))
 (segment (start 142.544802 92.6592) (end 143.814802 91.3892) (width 0.2) (layer "F.Cu") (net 15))
 (segment (start 129.06 82.31) (end 129.82 83.07) (width 0.2) (layer "F.Cu") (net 27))
 (segment (start 135.766 84.96) (end 136.194801 84.531199) (width 0.2) (layer "F.Cu") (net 27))
 (segment (start 119.66575 79.95285) (end 120.7516 81.0387) (width 0.2) (layer "F.Cu") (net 27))
 (segment (start 129.82 83.07) (end 129.82 84.393) (width 0.2) (layer "F.Cu") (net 27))
 (segment (start 129.82 84.393) (end 130.387 84.96) (width 0.2) (layer "F.Cu") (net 27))
 (segment (start 126.75 82.31) (end 129.06 82.31) (width 0.2) (layer "F.Cu") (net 27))
 (segment (start 130.387 84.96) (end 135.766 84.96) (width 0.2) (layer "F.Cu") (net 27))
 (segment (start 136.194801 84.531199) (end 136.194801 83.7692) (width 0.2) (layer "F.Cu") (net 27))
 (segment (start 120.7516 81.0387) (end 121.3387 81.0387) (width 0.2) (layer "F.Cu") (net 27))
 (segment (start 121.3387 81.0387) (end 121.83 81.53) (width 0.2) (layer "F.Cu") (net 27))
 (segment (start 121.83 81.53) (end 125.97 81.53) (width 0.2) (layer "F.Cu") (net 27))
 (segment (start 125.97 81.53) (end 126.75 82.31) (width 0.2) (layer "F.Cu") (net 27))
 (segment (start 141.2748 91.921148) (end 141.2748 91.3892) (width 0.2) (layer "B.Cu") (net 16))
 (segment (start 139.98575 95.19285) (end 139.98575 93.210198) (width 0.2) (layer "B.Cu") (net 16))
 (segment (start 139.98575 93.210198) (end 141.2748 91.921148) (width 0.2) (layer "B.Cu") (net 16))
 (segment (start 132.6388 78.232) (end 118.8466 78.232) (width 0.2) (layer "F.Cu") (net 28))
 (segment (start 133.654801 79.248001) (end 132.6388 78.232) (width 0.2) (layer "F.Cu") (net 28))
 (segment (start 133.654801 81.2292) (end 133.654801 79.248001) (width 0.2) (layer "F.Cu") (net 28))
 (segment (start 118.8466 78.232) (end 117.12575 79.95285) (width 0.2) (layer "F.Cu") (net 28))
 (segment (start 124.7648 85.1916) (end 125.0696 84.8868) (width 0.2) (layer "F.Cu") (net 5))
 (segment (start 122.0216 83.566) (end 123.6472 85.1916) (width 0.2) (layer "F.Cu") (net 5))
 (segment (start 123.6472 85.1916) (end 124.7648 85.1916) (width 0.2) (layer "F.Cu") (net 5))
 (segment (start 126.38 88.83) (end 126.38 86.8068) (width 0.2) (layer "F.Cu") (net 5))
 (segment (start 126.38 86.8068) (end 124.7648 85.1916) (width 0.2) (layer "F.Cu") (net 5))
 (via (at 126.38 88.83) (size 0.6) (drill 0.4) (layers "F.Cu" "B.Cu") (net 5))
 (segment (start 126.38 88.83) (end 126.38 89.194399) (width 0.2) (layer "B.Cu") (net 5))
 (segment (start 122.0216 83.566) (end 119.4308 83.566) (width 0.2) (layer "B.Cu") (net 5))
 (segment (start 126.38 89.194399) (end 128.574801 91.3892) (width 0.2) (layer "B.Cu") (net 5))
 (segment (start 127.5064 90.07) (end 129.894001 90.07) (width 0.2) (layer "F.Cu") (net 2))
 (segment (start 123.1392 91.186) (end 122.0216 91.186) (width 0.2) (layer "F.Cu") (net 2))
 (segment (start 129.894001 90.07) (end 131.114801 88.8492) (width 0.2) (layer "F.Cu") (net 2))
 (segment (start 124.7648 92.8116) (end 127.5064 90.07) (width 0.2) (layer "F.Cu") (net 2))
 (segment (start 124.7648 92.8116) (end 123.1392 91.186) (width 0.2) (layer "F.Cu") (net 2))
 (segment (start 122.0216 91.186) (end 119.4308 91.186) (width 0.2) (layer "B.Cu") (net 2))
 (segment (start 124.7648 90.2716) (end 123.1392 88.646) (width 0.2) (layer "F.Cu") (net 3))
 (segment (start 126.0184 90.2716) (end 124.7648 90.2716) (width 0.25) (layer "F.Cu") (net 3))
 (segment (start 127.05 85.87) (end 127.05 89.24) (width 0.25) (layer "F.Cu") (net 3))
 (segment (start 127.05 89.24) (end 126.0184 90.2716) (width 0.25) (layer "F.Cu") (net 3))
 (segment (start 123.1392 88.646) (end 122.0216 88.646) (width 0.2) (layer "F.Cu") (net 3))
 (via (at 127.05 85.87) (size 0.6) (drill 0.4) (layers "F.Cu" "B.Cu") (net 3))
 (segment (start 122.0216 88.646) (end 119.4308 88.646) (width 0.2) (layer "B.Cu") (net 3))
 (segment (start 125.0696 89.9668) (end 124.7648 90.2716) (width 0.2) (layer "B.Cu") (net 3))
 (segment (start 128.530799 81.229201) (end 127.31 82.45) (width 0.25) (layer "B.Cu") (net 3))
 (segment (start 127.31 82.45) (end 127.05 82.71) (width 0.25) (layer "B.Cu") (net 3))
 (segment (start 127.05 82.71) (end 127.05 85.87) (width 0.25) (layer "B.Cu") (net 3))
 (segment (start 131.114801 81.229201) (end 128.530799 81.229201) (width 0.25) (layer "B.Cu") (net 3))
 (segment (start 122.4788 86.106) (end 122.0216 86.106) (width 0.2) (layer "F.Cu") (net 4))
 (segment (start 123.3932 87.0204) (end 122.4788 86.106) (width 0.2) (layer "F.Cu") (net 4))
 (segment (start 124.7648 87.7316) (end 124.0536 87.0204) (width 0.2) (layer "F.Cu") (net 4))
 (segment (start 124.0536 87.0204) (end 123.3932 87.0204) (width 0.2) (layer "F.Cu") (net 4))
 (segment (start 132.86 84.564001) (end 132.86 87.45) (width 0.25) (layer "B.Cu") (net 4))
 (segment (start 122.0216 86.106) (end 119.4308 86.106) (width 0.2) (layer "B.Cu") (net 4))
 (segment (start 127.26 87.6) (end 127.1284 87.7316) (width 0.25) (layer "B.Cu") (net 4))
 (segment (start 132.86 87.45) (end 132.71 87.6) (width 0.25) (layer "B.Cu") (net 4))
 (segment (start 127.1284 87.7316) (end 124.7648 87.7316) (width 0.25) (layer "B.Cu") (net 4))
 (segment (start 133.654801 83.7692) (end 132.86 84.564001) (width 0.25) (layer "B.Cu") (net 4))
 (segment (start 132.71 87.6) (end 127.26 87.6) (width 0.25) (layer "B.Cu") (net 4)))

